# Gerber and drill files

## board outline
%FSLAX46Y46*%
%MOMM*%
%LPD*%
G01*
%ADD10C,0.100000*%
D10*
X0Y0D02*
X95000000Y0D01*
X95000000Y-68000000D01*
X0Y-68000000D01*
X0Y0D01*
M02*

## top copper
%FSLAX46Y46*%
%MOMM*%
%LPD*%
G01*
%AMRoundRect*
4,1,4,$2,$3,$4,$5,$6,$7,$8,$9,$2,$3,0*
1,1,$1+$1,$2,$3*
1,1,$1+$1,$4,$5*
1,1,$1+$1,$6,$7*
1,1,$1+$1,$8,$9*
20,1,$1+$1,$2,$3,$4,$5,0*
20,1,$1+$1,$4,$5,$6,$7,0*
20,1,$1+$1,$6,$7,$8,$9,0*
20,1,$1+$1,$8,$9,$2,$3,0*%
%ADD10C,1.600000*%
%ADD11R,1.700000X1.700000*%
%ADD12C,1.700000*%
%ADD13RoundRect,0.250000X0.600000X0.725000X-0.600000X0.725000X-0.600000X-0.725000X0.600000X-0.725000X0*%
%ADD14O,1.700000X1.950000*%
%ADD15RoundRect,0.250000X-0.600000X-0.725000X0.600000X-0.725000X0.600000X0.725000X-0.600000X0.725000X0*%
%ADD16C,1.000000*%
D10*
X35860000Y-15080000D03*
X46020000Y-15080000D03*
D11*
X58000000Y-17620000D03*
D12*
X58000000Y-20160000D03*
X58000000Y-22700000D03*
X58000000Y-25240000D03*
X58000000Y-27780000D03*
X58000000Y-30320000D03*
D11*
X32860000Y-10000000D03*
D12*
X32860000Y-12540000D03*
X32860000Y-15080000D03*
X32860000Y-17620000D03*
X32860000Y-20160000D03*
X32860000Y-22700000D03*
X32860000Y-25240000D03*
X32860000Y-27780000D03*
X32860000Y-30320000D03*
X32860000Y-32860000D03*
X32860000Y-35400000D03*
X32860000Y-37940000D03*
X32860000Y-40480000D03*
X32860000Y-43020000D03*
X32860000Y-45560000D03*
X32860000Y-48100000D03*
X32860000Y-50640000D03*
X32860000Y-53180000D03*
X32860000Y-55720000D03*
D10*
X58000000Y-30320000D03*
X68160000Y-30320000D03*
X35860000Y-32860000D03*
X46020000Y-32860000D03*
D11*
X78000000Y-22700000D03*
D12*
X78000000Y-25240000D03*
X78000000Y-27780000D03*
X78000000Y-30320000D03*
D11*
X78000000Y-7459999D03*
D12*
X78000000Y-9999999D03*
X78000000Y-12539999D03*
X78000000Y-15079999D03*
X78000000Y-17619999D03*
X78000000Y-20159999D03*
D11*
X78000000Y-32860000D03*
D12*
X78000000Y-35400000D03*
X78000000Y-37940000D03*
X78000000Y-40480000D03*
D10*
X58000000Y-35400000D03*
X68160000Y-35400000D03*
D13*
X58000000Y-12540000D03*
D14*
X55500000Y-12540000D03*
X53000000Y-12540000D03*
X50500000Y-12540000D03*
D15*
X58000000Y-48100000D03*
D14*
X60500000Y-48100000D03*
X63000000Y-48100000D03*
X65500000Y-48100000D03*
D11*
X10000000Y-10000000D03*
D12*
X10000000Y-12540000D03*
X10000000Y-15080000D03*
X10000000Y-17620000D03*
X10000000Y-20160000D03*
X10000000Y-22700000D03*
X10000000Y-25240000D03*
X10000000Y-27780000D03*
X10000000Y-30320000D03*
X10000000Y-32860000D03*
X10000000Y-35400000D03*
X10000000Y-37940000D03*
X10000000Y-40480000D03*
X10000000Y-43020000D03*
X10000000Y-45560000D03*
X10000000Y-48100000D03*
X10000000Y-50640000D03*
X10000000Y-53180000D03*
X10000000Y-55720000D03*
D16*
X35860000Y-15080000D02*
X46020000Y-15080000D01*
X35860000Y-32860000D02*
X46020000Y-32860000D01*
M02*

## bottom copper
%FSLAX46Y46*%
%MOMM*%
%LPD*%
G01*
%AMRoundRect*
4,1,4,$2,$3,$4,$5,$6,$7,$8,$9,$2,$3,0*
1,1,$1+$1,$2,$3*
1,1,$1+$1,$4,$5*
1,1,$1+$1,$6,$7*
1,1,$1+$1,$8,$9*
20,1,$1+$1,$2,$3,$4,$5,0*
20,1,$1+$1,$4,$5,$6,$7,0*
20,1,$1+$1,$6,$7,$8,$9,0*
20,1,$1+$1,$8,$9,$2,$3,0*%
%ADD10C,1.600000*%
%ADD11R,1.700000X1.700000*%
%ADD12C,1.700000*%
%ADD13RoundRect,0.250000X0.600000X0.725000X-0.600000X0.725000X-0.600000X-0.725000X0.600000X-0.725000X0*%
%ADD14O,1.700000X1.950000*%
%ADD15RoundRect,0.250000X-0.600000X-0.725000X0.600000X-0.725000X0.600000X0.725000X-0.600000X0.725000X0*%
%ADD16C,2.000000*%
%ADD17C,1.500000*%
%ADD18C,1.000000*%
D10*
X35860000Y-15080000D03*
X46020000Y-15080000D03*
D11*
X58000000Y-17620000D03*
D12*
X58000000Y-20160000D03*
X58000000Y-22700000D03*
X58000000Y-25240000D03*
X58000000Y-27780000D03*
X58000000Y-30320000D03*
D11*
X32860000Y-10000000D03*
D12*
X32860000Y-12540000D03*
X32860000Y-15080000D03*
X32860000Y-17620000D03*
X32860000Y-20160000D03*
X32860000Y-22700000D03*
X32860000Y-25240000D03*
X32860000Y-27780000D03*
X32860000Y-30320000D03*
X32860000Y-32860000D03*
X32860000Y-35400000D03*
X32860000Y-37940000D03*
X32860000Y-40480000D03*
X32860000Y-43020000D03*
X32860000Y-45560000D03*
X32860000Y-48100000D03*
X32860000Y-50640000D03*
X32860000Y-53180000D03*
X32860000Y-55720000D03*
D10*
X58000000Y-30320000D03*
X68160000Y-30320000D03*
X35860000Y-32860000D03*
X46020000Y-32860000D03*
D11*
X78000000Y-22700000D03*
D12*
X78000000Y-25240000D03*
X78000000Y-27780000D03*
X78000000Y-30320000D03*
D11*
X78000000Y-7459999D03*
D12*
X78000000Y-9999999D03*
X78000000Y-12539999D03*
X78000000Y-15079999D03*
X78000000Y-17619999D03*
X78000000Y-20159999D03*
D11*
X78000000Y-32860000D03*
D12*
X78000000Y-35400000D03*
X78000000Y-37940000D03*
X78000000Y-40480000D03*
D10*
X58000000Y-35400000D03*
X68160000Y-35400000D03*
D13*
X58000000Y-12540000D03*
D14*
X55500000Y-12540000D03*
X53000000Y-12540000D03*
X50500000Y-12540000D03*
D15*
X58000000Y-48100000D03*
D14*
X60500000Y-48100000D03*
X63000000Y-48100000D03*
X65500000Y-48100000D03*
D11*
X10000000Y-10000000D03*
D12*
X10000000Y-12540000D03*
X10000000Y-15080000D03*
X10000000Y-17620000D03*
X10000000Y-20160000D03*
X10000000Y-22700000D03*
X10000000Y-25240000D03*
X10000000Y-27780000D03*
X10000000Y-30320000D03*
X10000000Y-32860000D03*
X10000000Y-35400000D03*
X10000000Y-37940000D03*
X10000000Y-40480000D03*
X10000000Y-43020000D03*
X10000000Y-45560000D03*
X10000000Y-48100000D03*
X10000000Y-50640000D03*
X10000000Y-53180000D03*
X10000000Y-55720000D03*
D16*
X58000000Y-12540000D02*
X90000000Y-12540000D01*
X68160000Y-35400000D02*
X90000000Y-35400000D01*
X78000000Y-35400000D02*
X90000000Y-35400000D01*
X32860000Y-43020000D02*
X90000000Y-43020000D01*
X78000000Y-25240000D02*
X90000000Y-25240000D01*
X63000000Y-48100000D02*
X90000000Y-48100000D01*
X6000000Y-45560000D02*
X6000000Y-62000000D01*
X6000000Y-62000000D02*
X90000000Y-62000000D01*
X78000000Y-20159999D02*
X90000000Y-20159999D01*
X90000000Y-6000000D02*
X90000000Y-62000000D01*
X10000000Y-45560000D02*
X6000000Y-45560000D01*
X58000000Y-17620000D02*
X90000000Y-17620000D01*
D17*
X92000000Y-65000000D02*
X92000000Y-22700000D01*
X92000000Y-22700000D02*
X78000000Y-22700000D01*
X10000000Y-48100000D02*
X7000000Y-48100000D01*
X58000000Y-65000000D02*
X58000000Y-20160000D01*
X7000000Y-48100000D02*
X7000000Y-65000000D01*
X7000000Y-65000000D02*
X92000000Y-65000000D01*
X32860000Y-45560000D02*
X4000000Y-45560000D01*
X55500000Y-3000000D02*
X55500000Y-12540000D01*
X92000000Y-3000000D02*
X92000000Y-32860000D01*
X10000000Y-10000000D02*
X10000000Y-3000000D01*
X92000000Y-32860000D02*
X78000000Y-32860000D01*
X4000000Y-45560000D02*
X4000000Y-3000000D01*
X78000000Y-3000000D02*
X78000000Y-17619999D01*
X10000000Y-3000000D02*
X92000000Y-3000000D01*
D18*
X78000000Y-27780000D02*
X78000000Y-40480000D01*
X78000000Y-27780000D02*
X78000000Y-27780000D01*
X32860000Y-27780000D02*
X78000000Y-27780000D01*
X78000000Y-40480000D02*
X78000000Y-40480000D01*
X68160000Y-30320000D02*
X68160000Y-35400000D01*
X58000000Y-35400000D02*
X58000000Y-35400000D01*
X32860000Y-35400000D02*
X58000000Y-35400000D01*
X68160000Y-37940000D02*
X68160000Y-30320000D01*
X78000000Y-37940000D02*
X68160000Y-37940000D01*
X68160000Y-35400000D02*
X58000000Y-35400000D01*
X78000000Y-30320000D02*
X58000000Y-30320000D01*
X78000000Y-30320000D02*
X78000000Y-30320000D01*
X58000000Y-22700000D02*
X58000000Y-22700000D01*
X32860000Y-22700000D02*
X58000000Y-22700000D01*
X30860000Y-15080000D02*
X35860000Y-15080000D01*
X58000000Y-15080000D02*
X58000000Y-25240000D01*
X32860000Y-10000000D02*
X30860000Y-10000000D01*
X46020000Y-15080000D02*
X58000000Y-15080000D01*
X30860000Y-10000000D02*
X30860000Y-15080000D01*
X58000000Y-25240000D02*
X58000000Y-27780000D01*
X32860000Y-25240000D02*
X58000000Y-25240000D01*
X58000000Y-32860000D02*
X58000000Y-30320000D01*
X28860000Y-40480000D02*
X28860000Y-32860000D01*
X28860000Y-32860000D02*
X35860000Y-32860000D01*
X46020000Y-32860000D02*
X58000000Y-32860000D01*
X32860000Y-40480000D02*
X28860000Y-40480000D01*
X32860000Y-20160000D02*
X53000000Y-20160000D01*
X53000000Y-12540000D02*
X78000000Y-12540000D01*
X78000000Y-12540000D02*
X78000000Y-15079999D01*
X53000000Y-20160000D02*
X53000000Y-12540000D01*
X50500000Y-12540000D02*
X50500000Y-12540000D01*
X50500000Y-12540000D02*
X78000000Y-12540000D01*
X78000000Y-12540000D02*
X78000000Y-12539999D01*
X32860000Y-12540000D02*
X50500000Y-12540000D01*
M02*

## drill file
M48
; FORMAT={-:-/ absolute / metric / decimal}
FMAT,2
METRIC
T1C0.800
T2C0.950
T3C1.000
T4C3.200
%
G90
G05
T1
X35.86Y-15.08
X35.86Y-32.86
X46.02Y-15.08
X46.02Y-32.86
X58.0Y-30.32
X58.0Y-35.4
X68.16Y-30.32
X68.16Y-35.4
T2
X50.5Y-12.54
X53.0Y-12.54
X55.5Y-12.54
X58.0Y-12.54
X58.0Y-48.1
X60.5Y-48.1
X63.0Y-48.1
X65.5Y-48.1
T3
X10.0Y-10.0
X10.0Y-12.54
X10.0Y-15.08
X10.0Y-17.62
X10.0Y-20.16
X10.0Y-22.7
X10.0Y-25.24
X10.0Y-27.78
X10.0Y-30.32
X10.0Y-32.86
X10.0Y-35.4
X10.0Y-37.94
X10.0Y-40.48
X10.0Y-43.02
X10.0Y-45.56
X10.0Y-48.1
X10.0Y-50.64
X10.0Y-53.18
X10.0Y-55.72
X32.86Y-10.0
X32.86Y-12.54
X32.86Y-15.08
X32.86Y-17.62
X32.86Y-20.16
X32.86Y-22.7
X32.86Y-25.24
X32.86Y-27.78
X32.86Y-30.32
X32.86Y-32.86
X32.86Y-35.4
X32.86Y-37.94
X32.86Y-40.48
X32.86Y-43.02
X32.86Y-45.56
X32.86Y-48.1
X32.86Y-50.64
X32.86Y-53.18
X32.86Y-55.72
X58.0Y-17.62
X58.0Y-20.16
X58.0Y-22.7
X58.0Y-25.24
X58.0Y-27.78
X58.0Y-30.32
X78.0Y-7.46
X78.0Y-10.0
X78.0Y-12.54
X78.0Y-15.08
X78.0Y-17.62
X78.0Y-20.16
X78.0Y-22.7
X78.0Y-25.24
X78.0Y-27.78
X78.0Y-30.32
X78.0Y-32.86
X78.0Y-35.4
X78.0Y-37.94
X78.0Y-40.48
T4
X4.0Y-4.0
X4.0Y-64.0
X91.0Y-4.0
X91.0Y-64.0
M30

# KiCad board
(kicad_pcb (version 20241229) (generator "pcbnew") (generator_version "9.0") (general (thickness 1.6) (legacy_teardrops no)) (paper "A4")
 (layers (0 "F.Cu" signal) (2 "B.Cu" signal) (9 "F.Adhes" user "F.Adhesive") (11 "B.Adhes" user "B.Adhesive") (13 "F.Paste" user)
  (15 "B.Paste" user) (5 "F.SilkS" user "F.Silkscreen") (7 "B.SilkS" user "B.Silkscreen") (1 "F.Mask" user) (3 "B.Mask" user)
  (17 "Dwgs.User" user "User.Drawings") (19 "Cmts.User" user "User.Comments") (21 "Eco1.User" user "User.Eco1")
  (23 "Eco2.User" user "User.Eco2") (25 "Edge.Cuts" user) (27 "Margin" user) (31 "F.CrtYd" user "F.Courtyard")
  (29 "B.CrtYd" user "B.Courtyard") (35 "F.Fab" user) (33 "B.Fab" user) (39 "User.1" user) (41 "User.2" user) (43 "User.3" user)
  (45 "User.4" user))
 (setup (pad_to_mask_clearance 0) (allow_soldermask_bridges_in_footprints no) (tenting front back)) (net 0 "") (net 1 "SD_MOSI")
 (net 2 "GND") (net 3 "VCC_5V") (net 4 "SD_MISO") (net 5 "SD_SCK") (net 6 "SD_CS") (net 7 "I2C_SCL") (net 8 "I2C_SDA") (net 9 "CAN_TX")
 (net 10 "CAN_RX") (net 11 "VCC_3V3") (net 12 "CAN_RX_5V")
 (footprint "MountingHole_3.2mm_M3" (layer "F.Cu") (at 4 64)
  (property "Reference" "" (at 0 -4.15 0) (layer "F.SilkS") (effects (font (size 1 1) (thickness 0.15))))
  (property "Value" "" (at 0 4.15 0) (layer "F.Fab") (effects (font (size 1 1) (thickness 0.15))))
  (pad "" np_thru_hole circle (at 0 0) (size 3.2 3.2) (drill 3.2) (layers "*.Cu" "*.Mask")))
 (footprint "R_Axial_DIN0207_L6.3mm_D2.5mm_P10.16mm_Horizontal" (layer "F.Cu") (at 35.86 15.08)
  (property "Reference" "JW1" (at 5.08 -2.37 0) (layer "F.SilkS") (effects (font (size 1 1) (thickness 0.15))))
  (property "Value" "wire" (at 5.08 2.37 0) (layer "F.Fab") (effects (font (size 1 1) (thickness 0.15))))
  (pad "1" thru_hole circle (at 0 0) (size 1.6 1.6) (drill 0.8) (layers "*.Cu" "*.Mask") (remove_unused_layers no) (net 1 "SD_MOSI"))
  (pad "2" thru_hole circle (at 10.16 0) (size 1.6 1.6) (drill 0.8) (layers "*.Cu" "*.Mask") (remove_unused_layers no) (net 1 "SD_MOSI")))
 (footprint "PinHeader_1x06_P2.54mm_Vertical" (layer "F.Cu") (at 58 17.62)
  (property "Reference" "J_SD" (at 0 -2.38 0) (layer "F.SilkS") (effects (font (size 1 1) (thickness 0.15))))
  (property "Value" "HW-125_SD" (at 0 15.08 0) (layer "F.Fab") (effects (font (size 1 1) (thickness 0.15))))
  (pad "1" thru_hole rect (at 0 0) (size 1.7 1.7) (drill 1) (layers "*.Cu" "*.Mask") (remove_unused_layers no) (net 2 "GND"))
  (pad "2" thru_hole circle (at 0 2.54) (size 1.7 1.7) (drill 1) (layers "*.Cu" "*.Mask") (remove_unused_layers no) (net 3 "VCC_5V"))
  (pad "3" thru_hole circle (at 0 5.08) (size 1.7 1.7) (drill 1) (layers "*.Cu" "*.Mask") (remove_unused_layers no) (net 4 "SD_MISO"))
  (pad "4" thru_hole circle (at 0 7.62) (size 1.7 1.7) (drill 1) (layers "*.Cu" "*.Mask") (remove_unused_layers no) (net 1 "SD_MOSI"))
  (pad "5" thru_hole circle (at 0 10.16) (size 1.7 1.7) (drill 1) (layers "*.Cu" "*.Mask") (remove_unused_layers no) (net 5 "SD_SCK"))
  (pad "6" thru_hole circle (at 0 12.7) (size 1.7 1.7) (drill 1) (layers "*.Cu" "*.Mask") (remove_unused_layers no) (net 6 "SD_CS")))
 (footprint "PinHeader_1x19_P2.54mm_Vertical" (layer "F.Cu") (at 32.86 10)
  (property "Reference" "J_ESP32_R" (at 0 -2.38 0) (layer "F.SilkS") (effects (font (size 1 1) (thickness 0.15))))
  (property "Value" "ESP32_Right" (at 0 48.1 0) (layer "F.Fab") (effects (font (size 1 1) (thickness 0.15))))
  (pad "1" thru_hole rect (at 0 0) (size 1.7 1.7) (drill 1) (layers "*.Cu" "*.Mask") (remove_unused_layers no) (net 1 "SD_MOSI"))
  (pad "2" thru_hole circle (at 0 2.54) (size 1.7 1.7) (drill 1) (layers "*.Cu" "*.Mask") (remove_unused_layers no) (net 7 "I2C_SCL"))
  (pad "3" thru_hole circle (at 0 5.08) (size 1.7 1.7) (drill 1) (layers "*.Cu" "*.Mask") (remove_unused_layers no))
  (pad "4" thru_hole circle (at 0 7.62) (size 1.7 1.7) (drill 1) (layers "*.Cu" "*.Mask") (remove_unused_layers no))
  (pad "5" thru_hole circle (at 0 10.16) (size 1.7 1.7) (drill 1) (layers "*.Cu" "*.Mask") (remove_unused_layers no) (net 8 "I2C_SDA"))
  (pad "6" thru_hole circle (at 0 12.7) (size 1.7 1.7) (drill 1) (layers "*.Cu" "*.Mask") (remove_unused_layers no) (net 4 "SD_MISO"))
  (pad "7" thru_hole circle (at 0 15.24) (size 1.7 1.7) (drill 1) (layers "*.Cu" "*.Mask") (remove_unused_layers no) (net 5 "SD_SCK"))
  (pad "8" thru_hole circle (at 0 17.78) (size 1.7 1.7) (drill 1) (layers "*.Cu" "*.Mask") (remove_unused_layers no) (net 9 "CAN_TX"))
  (pad "9" thru_hole circle (at 0 20.32) (size 1.7 1.7) (drill 1) (layers "*.Cu" "*.Mask") (remove_unused_layers no))
  (pad "10" thru_hole circle (at 0 22.86) (size 1.7 1.7) (drill 1) (layers "*.Cu" "*.Mask") (remove_unused_layers no))
  (pad "11" thru_hole circle (at 0 25.4) (size 1.7 1.7) (drill 1) (layers "*.Cu" "*.Mask") (remove_unused_layers no) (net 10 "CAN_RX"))
  (pad "12" thru_hole circle (at 0 27.94) (size 1.7 1.7) (drill 1) (layers "*.Cu" "*.Mask") (remove_unused_layers no))
  (pad "13" thru_hole circle (at 0 30.48) (size 1.7 1.7) (drill 1) (layers "*.Cu" "*.Mask") (remove_unused_layers no) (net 6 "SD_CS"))
  (pad "14" thru_hole circle (at 0 33.02) (size 1.7 1.7) (drill 1) (layers "*.Cu" "*.Mask") (remove_unused_layers no) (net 2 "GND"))
  (pad "15" thru_hole circle (at 0 35.56) (size 1.7 1.7) (drill 1) (layers "*.Cu" "*.Mask") (remove_unused_layers no) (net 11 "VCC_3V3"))
  (pad "16" thru_hole circle (at 0 38.1) (size 1.7 1.7) (drill 1) (layers "*.Cu" "*.Mask") (remove_unused_layers no))
  (pad "17" thru_hole circle (at 0 40.64) (size 1.7 1.7) (drill 1) (layers "*.Cu" "*.Mask") (remove_unused_layers no))
  (pad "18" thru_hole circle (at 0 43.18) (size 1.7 1.7) (drill 1) (layers "*.Cu" "*.Mask") (remove_unused_layers no))
  (pad "19" thru_hole circle (at 0 45.72) (size 1.7 1.7) (drill 1) (layers "*.Cu" "*.Mask") (remove_unused_layers no)))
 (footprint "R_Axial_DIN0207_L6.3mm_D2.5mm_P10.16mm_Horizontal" (layer "F.Cu") (at 58 30.32)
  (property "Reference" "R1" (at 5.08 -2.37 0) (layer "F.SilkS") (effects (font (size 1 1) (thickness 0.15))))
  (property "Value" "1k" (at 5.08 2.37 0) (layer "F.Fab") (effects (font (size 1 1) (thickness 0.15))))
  (pad "1" thru_hole circle (at 0 0) (size 1.6 1.6) (drill 0.8) (layers "*.Cu" "*.Mask") (remove_unused_layers no) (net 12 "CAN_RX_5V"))
  (pad "2" thru_hole circle (at 10.16 0) (size 1.6 1.6) (drill 0.8) (layers "*.Cu" "*.Mask") (remove_unused_layers no) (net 10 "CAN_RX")))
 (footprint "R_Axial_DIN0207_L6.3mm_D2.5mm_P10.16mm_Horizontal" (layer "F.Cu") (at 35.86 32.86)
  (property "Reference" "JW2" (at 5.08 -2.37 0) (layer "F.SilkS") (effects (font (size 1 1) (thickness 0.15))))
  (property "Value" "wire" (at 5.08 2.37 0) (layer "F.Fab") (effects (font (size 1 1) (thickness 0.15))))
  (pad "1" thru_hole circle (at 0 0) (size 1.6 1.6) (drill 0.8) (layers "*.Cu" "*.Mask") (remove_unused_layers no) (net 6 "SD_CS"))
  (pad "2" thru_hole circle (at 10.16 0) (size 1.6 1.6) (drill 0.8) (layers "*.Cu" "*.Mask") (remove_unused_layers no) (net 6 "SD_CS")))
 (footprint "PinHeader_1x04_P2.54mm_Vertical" (layer "F.Cu") (at 78 22.7)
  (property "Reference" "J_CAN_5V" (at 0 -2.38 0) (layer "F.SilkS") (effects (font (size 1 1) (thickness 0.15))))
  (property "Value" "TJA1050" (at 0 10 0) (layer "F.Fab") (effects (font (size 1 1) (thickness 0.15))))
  (pad "1" thru_hole rect (at 0 0) (size 1.7 1.7) (drill 1) (layers "*.Cu" "*.Mask") (remove_unused_layers no) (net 3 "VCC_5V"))
  (pad "2" thru_hole circle (at 0 2.54) (size 1.7 1.7) (drill 1) (layers "*.Cu" "*.Mask") (remove_unused_layers no) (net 2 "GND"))
  (pad "3" thru_hole circle (at 0 5.08) (size 1.7 1.7) (drill 1) (layers "*.Cu" "*.Mask") (remove_unused_layers no) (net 9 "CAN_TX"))
  (pad "4" thru_hole circle (at 0 7.62) (size 1.7 1.7) (drill 1) (layers "*.Cu" "*.Mask") (remove_unused_layers no) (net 12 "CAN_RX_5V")))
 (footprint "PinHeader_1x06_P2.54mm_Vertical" (layer "F.Cu") (at 78 7.459999)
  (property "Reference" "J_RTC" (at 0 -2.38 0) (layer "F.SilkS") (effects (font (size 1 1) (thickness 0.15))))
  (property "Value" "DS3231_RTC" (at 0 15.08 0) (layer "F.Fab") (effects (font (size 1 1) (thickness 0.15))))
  (pad "1" thru_hole rect (at 0 0) (size 1.7 1.7) (drill 1) (layers "*.Cu" "*.Mask") (remove_unused_layers no))
  (pad "2" thru_hole circle (at 0 2.54) (size 1.7 1.7) (drill 1) (layers "*.Cu" "*.Mask") (remove_unused_layers no))
  (pad "3" thru_hole circle (at 0 5.08) (size 1.7 1.7) (drill 1) (layers "*.Cu" "*.Mask") (remove_unused_layers no) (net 7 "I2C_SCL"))
  (pad "4" thru_hole circle (at 0 7.62) (size 1.7 1.7) (drill 1) (layers "*.Cu" "*.Mask") (remove_unused_layers no) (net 8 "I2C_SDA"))
  (pad "5" thru_hole circle (at 0 10.16) (size 1.7 1.7) (drill 1) (layers "*.Cu" "*.Mask") (remove_unused_layers no) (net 11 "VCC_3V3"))
  (pad "6" thru_hole circle (at 0 12.7) (size 1.7 1.7) (drill 1) (layers "*.Cu" "*.Mask") (remove_unused_layers no) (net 2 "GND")))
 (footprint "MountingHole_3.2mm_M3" (layer "F.Cu") (at 91 64)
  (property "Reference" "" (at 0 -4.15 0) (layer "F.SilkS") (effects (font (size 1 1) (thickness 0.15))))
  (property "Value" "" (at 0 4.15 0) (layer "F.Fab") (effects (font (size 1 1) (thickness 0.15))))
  (pad "" np_thru_hole circle (at 0 0) (size 3.2 3.2) (drill 3.2) (layers "*.Cu" "*.Mask")))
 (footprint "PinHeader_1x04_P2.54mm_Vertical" (layer "F.Cu") (at 78 32.86)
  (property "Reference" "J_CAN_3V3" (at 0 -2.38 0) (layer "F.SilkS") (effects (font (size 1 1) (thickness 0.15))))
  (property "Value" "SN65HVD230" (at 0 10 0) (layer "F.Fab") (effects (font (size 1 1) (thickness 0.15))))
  (pad "1" thru_hole rect (at 0 0) (size 1.7 1.7) (drill 1) (layers "*.Cu" "*.Mask") (remove_unused_layers no) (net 11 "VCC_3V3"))
  (pad "2" thru_hole circle (at 0 2.54) (size 1.7 1.7) (drill 1) (layers "*.Cu" "*.Mask") (remove_unused_layers no) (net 2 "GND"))
  (pad "3" thru_hole circle (at 0 5.08) (size 1.7 1.7) (drill 1) (layers "*.Cu" "*.Mask") (remove_unused_layers no) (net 10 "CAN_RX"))
  (pad "4" thru_hole circle (at 0 7.62) (size 1.7 1.7) (drill 1) (layers "*.Cu" "*.Mask") (remove_unused_layers no) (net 9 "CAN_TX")))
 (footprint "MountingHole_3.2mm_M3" (layer "F.Cu") (at 4 4)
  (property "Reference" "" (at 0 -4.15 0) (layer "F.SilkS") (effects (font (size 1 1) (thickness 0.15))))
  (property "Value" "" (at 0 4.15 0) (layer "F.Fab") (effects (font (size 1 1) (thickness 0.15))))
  (pad "" np_thru_hole circle (at 0 0) (size 3.2 3.2) (drill 3.2) (layers "*.Cu" "*.Mask")))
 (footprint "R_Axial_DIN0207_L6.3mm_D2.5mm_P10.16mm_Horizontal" (layer "F.Cu") (at 58 35.4)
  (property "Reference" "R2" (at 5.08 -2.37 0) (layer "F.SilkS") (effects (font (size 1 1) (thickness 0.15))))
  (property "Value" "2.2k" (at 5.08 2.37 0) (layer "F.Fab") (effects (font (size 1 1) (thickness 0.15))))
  (pad "1" thru_hole circle (at 0 0) (size 1.6 1.6) (drill 0.8) (layers "*.Cu" "*.Mask") (remove_unused_layers no) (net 10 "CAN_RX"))
  (pad "2" thru_hole circle (at 10.16 0) (size 1.6 1.6) (drill 0.8) (layers "*.Cu" "*.Mask") (remove_unused_layers no) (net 2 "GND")))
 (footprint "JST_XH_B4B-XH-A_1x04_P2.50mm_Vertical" (layer "F.Cu") (at 58 12.54 180)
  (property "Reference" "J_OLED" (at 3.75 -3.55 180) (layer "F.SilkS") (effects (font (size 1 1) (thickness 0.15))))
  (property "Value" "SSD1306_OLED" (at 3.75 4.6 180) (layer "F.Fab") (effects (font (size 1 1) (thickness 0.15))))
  (pad "1" thru_hole roundrect (at 0 0 180) (size 1.7 1.95) (drill 0.95) (layers "*.Cu" "*.Mask") (remove_unused_layers no)
   (roundrect_rratio 0.147059) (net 2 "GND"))
  (pad "2" thru_hole oval (at 2.5 0 180) (size 1.7 1.95) (drill 0.95) (layers "*.Cu" "*.Mask") (remove_unused_layers no) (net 11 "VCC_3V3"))
  (pad "3" thru_hole oval (at 5 0 180) (size 1.7 1.95) (drill 0.95) (layers "*.Cu" "*.Mask") (remove_unused_layers no) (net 8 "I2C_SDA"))
  (pad "4" thru_hole oval (at 7.5 0 180) (size 1.7 1.95) (drill 0.95) (layers "*.Cu" "*.Mask") (remove_unused_layers no) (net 7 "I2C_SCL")))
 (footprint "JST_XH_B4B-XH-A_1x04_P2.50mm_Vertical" (layer "F.Cu") (at 58 48.1)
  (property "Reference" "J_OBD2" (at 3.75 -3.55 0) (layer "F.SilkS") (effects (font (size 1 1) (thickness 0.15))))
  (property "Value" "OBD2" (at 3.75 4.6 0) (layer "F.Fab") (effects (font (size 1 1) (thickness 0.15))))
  (pad "1" thru_hole roundrect (at 0 0) (size 1.7 1.95) (drill 0.95) (layers "*.Cu" "*.Mask") (remove_unused_layers no)
   (roundrect_rratio 0.147059))
  (pad "2" thru_hole oval (at 2.5 0) (size 1.7 1.95) (drill 0.95) (layers "*.Cu" "*.Mask") (remove_unused_layers no))
  (pad "3" thru_hole oval (at 5 0) (size 1.7 1.95) (drill 0.95) (layers "*.Cu" "*.Mask") (remove_unused_layers no) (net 2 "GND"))
  (pad "4" thru_hole oval (at 7.5 0) (size 1.7 1.95) (drill 0.95) (layers "*.Cu" "*.Mask") (remove_unused_layers no)))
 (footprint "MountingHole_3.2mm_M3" (layer "F.Cu") (at 91 4)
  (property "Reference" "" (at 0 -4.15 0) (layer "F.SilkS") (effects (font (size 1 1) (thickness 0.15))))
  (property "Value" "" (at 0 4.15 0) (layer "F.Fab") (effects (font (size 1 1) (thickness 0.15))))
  (pad "" np_thru_hole circle (at 0 0) (size 3.2 3.2) (drill 3.2) (layers "*.Cu" "*.Mask")))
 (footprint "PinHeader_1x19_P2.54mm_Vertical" (layer "F.Cu") (at 10 10)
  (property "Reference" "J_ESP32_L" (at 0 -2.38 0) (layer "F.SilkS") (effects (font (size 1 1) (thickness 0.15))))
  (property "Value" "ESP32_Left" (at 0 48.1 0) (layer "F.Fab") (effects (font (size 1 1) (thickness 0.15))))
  (pad "1" thru_hole rect (at 0 0) (size 1.7 1.7) (drill 1) (layers "*.Cu" "*.Mask") (remove_unused_layers no) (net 11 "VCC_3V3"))
  (pad "2" thru_hole circle (at 0 2.54) (size 1.7 1.7) (drill 1) (layers "*.Cu" "*.Mask") (remove_unused_layers no))
  (pad "3" thru_hole circle (at 0 5.08) (size 1.7 1.7) (drill 1) (layers "*.Cu" "*.Mask") (remove_unused_layers no))
  (pad "4" thru_hole circle (at 0 7.62) (size 1.7 1.7) (drill 1) (layers "*.Cu" "*.Mask") (remove_unused_layers no))
  (pad "5" thru_hole circle (at 0 10.16) (size 1.7 1.7) (drill 1) (layers "*.Cu" "*.Mask") (remove_unused_layers no))
  (pad "6" thru_hole circle (at 0 12.7) (size 1.7 1.7) (drill 1) (layers "*.Cu" "*.Mask") (remove_unused_layers no))
  (pad "7" thru_hole circle (at 0 15.24) (size 1.7 1.7) (drill 1) (layers "*.Cu" "*.Mask") (remove_unused_layers no))
  (pad "8" thru_hole circle (at 0 17.78) (size 1.7 1.7) (drill 1) (layers "*.Cu" "*.Mask") (remove_unused_layers no))
  (pad "9" thru_hole circle (at 0 20.32) (size 1.7 1.7) (drill 1) (layers "*.Cu" "*.Mask") (remove_unused_layers no))
  (pad "10" thru_hole circle (at 0 22.86) (size 1.7 1.7) (drill 1) (layers "*.Cu" "*.Mask") (remove_unused_layers no))
  (pad "11" thru_hole circle (at 0 25.4) (size 1.7 1.7) (drill 1) (layers "*.Cu" "*.Mask") (remove_unused_layers no))
  (pad "12" thru_hole circle (at 0 27.94) (size 1.7 1.7) (drill 1) (layers "*.Cu" "*.Mask") (remove_unused_layers no))
  (pad "13" thru_hole circle (at 0 30.48) (size 1.7 1.7) (drill 1) (layers "*.Cu" "*.Mask") (remove_unused_layers no))
  (pad "14" thru_hole circle (at 0 33.02) (size 1.7 1.7) (drill 1) (layers "*.Cu" "*.Mask") (remove_unused_layers no))
  (pad "15" thru_hole circle (at 0 35.56) (size 1.7 1.7) (drill 1) (layers "*.Cu" "*.Mask") (remove_unused_layers no) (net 2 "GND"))
  (pad "16" thru_hole circle (at 0 38.1) (size 1.7 1.7) (drill 1) (layers "*.Cu" "*.Mask") (remove_unused_layers no) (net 3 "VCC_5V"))
  (pad "17" thru_hole circle (at 0 40.64) (size 1.7 1.7) (drill 1) (layers "*.Cu" "*.Mask") (remove_unused_layers no))
  (pad "18" thru_hole circle (at 0 43.18) (size 1.7 1.7) (drill 1) (layers "*.Cu" "*.Mask") (remove_unused_layers no))
  (pad "19" thru_hole circle (at 0 45.72) (size 1.7 1.7) (drill 1) (layers "*.Cu" "*.Mask") (remove_unused_layers no)))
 (gr_rect (start 0 0) (end 95 68) (stroke (width 0.1) (type default)) (fill no) (layer "Edge.Cuts"))
 (segment (start 58 12.54) (end 90 12.54) (width 2) (layer "B.Cu") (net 2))
 (segment (start 68.16 35.4) (end 90 35.4) (width 2) (layer "B.Cu") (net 2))
 (segment (start 78 35.4) (end 90 35.4) (width 2) (layer "B.Cu") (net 2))
 (segment (start 32.86 43.02) (end 90 43.02) (width 2) (layer "B.Cu") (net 2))
 (segment (start 78 25.24) (end 90 25.24) (width 2) (layer "B.Cu") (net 2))
 (segment (start 63 48.1) (end 90 48.1) (width 2) (layer "B.Cu") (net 2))
 (segment (start 6 45.56) (end 6 62) (width 2) (layer "B.Cu") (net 2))
 (segment (start 6 62) (end 90 62) (width 2) (layer "B.Cu") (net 2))
 (segment (start 78 20.159999) (end 90 20.159999) (width 2) (layer "B.Cu") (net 2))
 (segment (start 90 6) (end 90 62) (width 2) (layer "B.Cu") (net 2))
 (segment (start 10 45.56) (end 6 45.56) (width 2) (layer "B.Cu") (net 2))
 (segment (start 58 17.62) (end 90 17.62) (width 2) (layer "B.Cu") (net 2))
 (segment (start 92 65) (end 92 22.7) (width 1.5) (layer "B.Cu") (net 3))
 (segment (start 92 22.7) (end 78 22.7) (width 1.5) (layer "B.Cu") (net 3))
 (segment (start 10 48.1) (end 7 48.1) (width 1.5) (layer "B.Cu") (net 3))
 (segment (start 58 65) (end 58 20.16) (width 1.5) (layer "B.Cu") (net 3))
 (segment (start 7 48.1) (end 7 65) (width 1.5) (layer "B.Cu") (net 3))
 (segment (start 7 65) (end 92 65) (width 1.5) (layer "B.Cu") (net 3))
 (segment (start 32.86 45.56) (end 4 45.56) (width 1.5) (layer "B.Cu") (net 11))
 (segment (start 55.5 3) (end 55.5 12.54) (width 1.5) (layer "B.Cu") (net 11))
 (segment (start 92 3) (end 92 32.86) (width 1.5) (layer "B.Cu") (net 11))
 (segment (start 10 10) (end 10 3) (width 1.5) (layer "B.Cu") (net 11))
 (segment (start 92 32.86) (end 78 32.86) (width 1.5) (layer "B.Cu") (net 11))
 (segment (start 4 45.56) (end 4 3) (width 1.5) (layer "B.Cu") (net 11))
 (segment (start 78 3) (end 78 17.619999) (width 1.5) (layer "B.Cu") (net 11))
 (segment (start 10 3) (end 92 3) (width 1.5) (layer "B.Cu") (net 11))
 (segment (start 78 27.78) (end 78 40.48) (width 1) (layer "B.Cu") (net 9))
 (segment (start 78 27.78) (end 78 27.78) (width 1) (layer "B.Cu") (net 9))
 (segment (start 32.86 27.78) (end 78 27.78) (width 1) (layer "B.Cu") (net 9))
 (segment (start 78 40.48) (end 78 40.48) (width 1) (layer "B.Cu") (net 9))
 (segment (start 68.16 30.32) (end 68.16 35.4) (width 1) (layer "B.Cu") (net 10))
 (segment (start 58 35.4) (end 58 35.4) (width 1) (layer "B.Cu") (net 10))
 (segment (start 32.86 35.4) (end 58 35.4) (width 1) (layer "B.Cu") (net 10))
 (segment (start 68.16 37.94) (end 68.16 30.32) (width 1) (layer "B.Cu") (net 10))
 (segment (start 78 37.94) (end 68.16 37.94) (width 1) (layer "B.Cu") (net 10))
 (segment (start 68.16 35.4) (end 58 35.4) (width 1) (layer "B.Cu") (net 10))
 (segment (start 78 30.32) (end 58 30.32) (width 1) (layer "B.Cu") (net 12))
 (segment (start 78 30.32) (end 78 30.32) (width 1) (layer "B.Cu") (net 12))
 (segment (start 58 22.7) (end 58 22.7) (width 1) (layer "B.Cu") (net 4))
 (segment (start 32.86 22.7) (end 58 22.7) (width 1) (layer "B.Cu") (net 4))
 (segment (start 35.86 15.08) (end 46.02 15.08) (width 1) (layer "F.Cu") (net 1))
 (segment (start 30.86 15.08) (end 35.86 15.08) (width 1) (layer "B.Cu") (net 1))
 (segment (start 58 15.08) (end 58 25.24) (width 1) (layer "B.Cu") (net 1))
 (segment (start 32.86 10) (end 30.86 10) (width 1) (layer "B.Cu") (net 1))
 (segment (start 46.02 15.08) (end 58 15.08) (width 1) (layer "B.Cu") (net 1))
 (segment (start 30.86 10) (end 30.86 15.08) (width 1) (layer "B.Cu") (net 1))
 (segment (start 58 25.24) (end 58 27.78) (width 1) (layer "B.Cu") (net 5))
 (segment (start 32.86 25.24) (end 58 25.24) (width 1) (layer "B.Cu") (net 5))
 (segment (start 35.86 32.86) (end 46.02 32.86) (width 1) (layer "F.Cu") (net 6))
 (segment (start 58 32.86) (end 58 30.32) (width 1) (layer "B.Cu") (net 6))
 (segment (start 28.86 40.48) (end 28.86 32.86) (width 1) (layer "B.Cu") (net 6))
 (segment (start 28.86 32.86) (end 35.86 32.86) (width 1) (layer "B.Cu") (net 6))
 (segment (start 46.02 32.86) (end 58 32.86) (width 1) (layer "B.Cu") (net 6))
 (segment (start 32.86 40.48) (end 28.86 40.48) (width 1) (layer "B.Cu") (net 6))
 (segment (start 32.86 20.16) (end 53 20.16) (width 1) (layer "B.Cu") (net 8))
 (segment (start 53 12.54) (end 78 12.54) (width 1) (layer "B.Cu") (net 8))
 (segment (start 78 12.54) (end 78 15.079999) (width 1) (layer "B.Cu") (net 8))
 (segment (start 53 20.16) (end 53 12.54) (width 1) (layer "B.Cu") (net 8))
 (segment (start 50.5 12.54) (end 50.5 12.54) (width 1) (layer "B.Cu") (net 7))
 (segment (start 50.5 12.54) (end 78 12.54) (width 1) (layer "B.Cu") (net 7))
 (segment (start 78 12.54) (end 78 12.539999) (width 1) (layer "B.Cu") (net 7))
 (segment (start 32.86 12.54) (end 50.5 12.54) (width 1) (layer "B.Cu") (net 7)))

